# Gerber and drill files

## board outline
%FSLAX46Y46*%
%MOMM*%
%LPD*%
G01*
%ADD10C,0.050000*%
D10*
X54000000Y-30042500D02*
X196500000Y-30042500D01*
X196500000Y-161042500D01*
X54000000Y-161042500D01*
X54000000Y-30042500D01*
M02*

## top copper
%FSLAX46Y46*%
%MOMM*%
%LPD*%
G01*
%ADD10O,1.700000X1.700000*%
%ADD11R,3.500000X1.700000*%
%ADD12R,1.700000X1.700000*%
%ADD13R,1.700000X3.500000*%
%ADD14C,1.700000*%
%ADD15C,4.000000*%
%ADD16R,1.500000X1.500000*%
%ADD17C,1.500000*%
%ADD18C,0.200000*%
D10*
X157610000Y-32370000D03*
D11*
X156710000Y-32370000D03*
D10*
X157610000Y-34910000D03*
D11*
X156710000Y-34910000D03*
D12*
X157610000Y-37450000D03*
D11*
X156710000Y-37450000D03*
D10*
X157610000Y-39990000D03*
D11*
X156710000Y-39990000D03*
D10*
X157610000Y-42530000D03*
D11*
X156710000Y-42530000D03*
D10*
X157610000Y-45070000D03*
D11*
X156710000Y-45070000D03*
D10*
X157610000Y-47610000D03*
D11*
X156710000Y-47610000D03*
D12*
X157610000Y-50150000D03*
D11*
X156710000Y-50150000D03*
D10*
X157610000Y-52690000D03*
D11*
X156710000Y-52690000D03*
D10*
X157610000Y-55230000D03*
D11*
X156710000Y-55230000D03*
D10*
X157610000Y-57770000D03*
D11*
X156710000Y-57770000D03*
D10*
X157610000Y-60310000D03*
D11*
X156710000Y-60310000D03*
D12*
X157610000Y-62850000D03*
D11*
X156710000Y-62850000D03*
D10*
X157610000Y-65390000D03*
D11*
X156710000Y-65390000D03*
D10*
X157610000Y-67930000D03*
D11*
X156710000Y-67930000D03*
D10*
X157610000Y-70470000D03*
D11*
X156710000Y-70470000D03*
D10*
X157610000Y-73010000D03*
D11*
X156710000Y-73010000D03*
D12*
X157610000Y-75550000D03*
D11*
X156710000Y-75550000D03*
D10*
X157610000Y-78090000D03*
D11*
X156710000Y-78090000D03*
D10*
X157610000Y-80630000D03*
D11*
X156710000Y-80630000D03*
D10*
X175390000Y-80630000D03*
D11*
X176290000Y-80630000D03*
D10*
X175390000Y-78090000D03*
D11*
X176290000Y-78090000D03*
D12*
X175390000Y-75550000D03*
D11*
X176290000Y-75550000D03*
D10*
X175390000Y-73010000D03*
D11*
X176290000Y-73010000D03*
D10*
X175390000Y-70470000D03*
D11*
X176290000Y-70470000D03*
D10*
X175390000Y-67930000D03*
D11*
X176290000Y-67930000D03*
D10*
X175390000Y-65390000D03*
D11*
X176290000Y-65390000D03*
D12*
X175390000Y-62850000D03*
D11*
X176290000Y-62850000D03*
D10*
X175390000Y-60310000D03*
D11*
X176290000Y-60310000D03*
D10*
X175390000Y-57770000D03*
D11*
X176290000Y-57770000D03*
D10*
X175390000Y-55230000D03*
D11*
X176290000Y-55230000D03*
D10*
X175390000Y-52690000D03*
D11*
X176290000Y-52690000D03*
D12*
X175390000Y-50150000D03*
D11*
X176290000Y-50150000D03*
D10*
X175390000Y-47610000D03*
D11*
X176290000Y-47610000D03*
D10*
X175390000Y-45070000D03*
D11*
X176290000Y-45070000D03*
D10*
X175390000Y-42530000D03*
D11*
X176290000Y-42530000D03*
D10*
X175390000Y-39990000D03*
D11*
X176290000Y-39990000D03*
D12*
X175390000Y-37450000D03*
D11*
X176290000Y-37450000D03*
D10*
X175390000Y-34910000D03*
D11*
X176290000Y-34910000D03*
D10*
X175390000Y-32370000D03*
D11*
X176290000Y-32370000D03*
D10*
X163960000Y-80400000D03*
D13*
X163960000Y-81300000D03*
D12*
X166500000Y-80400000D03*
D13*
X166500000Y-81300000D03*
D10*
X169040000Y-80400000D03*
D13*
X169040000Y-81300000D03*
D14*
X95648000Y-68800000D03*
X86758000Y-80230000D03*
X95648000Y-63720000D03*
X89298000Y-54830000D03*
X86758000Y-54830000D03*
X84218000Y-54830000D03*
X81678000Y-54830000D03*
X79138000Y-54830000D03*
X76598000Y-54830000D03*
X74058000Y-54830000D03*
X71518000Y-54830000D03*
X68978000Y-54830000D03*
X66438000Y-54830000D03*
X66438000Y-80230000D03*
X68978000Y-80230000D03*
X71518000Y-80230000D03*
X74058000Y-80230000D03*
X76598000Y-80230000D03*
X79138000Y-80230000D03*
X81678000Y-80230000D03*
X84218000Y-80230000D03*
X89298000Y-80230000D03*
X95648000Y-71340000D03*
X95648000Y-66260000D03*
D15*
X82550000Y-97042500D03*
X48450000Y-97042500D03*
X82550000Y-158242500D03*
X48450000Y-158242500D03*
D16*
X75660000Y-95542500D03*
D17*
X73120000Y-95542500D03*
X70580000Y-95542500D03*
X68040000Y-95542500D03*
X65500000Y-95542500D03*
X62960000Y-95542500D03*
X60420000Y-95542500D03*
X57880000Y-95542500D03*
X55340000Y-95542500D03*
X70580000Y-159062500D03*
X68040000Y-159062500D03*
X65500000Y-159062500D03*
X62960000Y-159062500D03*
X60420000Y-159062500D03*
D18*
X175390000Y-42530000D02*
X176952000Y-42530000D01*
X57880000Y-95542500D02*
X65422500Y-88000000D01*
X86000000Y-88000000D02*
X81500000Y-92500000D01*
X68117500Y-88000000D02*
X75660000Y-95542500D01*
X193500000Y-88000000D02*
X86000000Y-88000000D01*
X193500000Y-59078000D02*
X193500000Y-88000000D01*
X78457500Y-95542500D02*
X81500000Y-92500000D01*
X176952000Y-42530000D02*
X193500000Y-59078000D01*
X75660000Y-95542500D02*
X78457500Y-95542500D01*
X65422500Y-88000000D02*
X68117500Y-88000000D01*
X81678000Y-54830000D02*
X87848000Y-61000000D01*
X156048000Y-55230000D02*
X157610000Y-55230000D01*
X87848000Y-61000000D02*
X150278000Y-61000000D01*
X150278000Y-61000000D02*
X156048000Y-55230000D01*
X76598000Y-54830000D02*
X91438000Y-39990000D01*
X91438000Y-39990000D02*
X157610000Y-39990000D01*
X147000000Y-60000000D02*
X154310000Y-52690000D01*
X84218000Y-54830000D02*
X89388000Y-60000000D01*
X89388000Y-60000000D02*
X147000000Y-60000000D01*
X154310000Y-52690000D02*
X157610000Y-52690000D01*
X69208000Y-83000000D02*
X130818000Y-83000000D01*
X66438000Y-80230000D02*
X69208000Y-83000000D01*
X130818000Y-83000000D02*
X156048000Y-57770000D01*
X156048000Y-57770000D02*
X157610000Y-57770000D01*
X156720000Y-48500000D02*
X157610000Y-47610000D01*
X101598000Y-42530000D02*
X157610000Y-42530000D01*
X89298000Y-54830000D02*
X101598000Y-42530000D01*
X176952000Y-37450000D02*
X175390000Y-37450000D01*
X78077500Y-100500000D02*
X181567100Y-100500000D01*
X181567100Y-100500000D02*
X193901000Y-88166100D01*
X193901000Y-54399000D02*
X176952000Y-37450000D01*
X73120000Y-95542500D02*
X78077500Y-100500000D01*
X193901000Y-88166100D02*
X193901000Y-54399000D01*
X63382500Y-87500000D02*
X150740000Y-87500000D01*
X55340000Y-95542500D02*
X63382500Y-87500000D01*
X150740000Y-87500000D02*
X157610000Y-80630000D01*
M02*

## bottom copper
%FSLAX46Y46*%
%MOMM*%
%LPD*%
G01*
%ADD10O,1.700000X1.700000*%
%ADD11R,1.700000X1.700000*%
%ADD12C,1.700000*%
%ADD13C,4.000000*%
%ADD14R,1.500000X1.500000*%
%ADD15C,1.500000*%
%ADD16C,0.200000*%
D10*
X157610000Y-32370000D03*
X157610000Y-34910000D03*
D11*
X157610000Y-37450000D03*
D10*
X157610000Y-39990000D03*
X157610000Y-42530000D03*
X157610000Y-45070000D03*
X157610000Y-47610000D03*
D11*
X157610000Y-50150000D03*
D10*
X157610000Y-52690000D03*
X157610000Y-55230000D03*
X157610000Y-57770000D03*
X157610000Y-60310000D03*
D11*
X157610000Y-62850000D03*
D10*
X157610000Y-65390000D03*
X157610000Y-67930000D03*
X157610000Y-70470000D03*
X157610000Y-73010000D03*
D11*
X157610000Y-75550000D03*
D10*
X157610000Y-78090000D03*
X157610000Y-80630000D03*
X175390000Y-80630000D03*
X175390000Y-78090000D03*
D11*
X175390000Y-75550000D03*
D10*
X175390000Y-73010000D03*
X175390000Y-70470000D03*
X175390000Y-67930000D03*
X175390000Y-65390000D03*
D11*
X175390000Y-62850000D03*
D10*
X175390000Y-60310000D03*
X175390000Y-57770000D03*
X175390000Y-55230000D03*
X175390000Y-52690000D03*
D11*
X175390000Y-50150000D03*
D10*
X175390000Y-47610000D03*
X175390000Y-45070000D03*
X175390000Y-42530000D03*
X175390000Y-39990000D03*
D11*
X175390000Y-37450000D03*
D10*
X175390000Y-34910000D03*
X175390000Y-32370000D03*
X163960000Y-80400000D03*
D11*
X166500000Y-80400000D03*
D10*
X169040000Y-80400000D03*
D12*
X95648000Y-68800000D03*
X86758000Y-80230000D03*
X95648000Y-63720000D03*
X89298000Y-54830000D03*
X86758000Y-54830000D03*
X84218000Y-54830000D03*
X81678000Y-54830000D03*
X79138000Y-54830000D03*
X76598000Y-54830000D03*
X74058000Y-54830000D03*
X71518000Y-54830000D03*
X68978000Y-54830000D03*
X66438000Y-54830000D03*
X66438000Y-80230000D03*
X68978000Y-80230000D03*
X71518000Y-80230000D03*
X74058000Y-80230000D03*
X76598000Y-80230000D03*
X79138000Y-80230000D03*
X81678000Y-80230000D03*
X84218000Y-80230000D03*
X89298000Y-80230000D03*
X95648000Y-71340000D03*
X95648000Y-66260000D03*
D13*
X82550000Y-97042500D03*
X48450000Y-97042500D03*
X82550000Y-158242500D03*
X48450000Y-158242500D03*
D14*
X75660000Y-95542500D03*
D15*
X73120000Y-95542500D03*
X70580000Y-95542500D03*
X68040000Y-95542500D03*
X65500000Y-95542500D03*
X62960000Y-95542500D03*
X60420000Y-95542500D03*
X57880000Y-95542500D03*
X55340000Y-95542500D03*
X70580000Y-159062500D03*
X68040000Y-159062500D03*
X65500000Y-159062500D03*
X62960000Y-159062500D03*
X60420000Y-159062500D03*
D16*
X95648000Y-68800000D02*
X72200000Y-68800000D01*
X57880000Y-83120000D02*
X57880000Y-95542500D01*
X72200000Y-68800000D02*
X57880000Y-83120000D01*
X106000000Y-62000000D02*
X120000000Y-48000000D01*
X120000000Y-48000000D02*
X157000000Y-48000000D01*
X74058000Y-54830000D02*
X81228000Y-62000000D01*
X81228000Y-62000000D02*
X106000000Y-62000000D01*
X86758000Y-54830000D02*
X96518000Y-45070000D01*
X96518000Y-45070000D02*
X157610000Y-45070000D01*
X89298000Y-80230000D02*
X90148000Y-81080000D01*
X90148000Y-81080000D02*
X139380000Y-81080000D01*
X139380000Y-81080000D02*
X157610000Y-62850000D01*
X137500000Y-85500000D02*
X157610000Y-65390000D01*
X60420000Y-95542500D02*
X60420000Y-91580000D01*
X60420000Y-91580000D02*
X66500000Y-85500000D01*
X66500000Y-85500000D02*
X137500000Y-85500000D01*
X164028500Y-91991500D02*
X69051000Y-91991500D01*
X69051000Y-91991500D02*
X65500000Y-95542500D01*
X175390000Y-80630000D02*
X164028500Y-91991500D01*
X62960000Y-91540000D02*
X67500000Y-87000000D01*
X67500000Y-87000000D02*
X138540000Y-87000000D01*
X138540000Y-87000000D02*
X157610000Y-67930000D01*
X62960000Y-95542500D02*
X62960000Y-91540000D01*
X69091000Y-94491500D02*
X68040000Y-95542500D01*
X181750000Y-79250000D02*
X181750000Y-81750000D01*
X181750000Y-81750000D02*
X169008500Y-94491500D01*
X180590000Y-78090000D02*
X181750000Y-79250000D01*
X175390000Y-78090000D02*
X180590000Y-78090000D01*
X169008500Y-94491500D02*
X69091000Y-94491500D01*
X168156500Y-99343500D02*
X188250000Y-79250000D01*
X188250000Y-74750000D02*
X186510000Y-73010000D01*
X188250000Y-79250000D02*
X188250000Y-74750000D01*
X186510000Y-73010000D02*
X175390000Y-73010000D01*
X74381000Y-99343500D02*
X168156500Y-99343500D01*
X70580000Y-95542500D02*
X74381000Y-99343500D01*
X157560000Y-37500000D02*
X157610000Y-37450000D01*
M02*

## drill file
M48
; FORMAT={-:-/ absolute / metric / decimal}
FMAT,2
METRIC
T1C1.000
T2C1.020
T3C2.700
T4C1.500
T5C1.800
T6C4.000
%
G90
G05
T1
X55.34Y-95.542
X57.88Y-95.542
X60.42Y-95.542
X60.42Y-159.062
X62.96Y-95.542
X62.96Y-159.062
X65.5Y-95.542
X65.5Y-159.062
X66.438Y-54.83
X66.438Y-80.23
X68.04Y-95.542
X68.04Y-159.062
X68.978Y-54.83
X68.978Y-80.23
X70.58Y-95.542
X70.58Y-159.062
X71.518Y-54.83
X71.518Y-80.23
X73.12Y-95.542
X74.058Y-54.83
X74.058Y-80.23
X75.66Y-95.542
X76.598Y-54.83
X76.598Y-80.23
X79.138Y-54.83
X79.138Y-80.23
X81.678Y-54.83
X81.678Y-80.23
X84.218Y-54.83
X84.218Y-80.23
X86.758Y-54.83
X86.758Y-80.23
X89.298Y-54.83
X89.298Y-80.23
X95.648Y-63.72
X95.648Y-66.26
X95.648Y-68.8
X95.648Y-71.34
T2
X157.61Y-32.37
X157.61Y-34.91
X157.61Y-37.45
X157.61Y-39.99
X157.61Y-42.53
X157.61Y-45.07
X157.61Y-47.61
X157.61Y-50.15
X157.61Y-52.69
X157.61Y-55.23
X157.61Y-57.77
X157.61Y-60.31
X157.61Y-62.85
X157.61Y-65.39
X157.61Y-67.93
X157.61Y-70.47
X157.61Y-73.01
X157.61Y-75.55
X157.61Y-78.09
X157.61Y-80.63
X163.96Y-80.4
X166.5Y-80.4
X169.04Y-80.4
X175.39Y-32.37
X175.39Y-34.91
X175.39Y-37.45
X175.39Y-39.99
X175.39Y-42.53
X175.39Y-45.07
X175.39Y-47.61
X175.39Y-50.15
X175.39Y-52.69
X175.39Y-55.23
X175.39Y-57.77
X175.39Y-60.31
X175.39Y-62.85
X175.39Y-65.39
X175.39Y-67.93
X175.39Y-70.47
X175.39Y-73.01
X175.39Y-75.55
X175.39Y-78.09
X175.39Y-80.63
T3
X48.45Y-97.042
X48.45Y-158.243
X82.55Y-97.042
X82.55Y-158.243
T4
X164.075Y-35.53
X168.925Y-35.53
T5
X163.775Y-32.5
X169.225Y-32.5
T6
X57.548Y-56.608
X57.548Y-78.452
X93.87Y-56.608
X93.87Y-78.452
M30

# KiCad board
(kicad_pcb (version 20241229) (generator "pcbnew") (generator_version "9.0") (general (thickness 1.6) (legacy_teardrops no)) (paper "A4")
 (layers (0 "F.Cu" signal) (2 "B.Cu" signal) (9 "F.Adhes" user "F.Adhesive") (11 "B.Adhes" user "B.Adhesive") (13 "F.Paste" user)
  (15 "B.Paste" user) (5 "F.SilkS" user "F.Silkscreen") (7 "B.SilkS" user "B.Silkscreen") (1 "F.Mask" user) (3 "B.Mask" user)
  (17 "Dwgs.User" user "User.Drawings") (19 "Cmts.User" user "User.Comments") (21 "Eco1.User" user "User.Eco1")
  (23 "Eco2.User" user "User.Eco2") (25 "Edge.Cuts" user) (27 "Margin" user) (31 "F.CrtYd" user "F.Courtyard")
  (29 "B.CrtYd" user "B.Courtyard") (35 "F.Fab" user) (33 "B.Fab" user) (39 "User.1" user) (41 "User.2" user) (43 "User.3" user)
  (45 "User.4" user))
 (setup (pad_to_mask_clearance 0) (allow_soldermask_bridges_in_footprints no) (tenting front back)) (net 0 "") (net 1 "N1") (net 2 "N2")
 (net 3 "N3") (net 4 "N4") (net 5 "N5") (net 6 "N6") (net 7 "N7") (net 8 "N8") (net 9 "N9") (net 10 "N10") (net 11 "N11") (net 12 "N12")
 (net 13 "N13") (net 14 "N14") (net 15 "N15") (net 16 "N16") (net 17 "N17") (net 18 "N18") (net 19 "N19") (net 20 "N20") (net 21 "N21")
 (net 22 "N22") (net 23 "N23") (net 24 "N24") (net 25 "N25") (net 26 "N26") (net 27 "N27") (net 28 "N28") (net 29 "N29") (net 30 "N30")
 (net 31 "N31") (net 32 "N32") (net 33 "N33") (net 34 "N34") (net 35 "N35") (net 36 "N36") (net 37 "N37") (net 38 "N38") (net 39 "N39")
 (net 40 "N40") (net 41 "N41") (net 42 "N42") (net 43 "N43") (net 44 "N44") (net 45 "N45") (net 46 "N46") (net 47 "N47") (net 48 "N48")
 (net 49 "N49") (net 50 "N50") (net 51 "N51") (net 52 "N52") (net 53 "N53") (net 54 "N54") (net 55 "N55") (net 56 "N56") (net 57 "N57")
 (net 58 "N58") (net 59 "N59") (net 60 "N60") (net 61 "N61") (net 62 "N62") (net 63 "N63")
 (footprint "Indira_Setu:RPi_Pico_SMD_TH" (layer "F.Cu") (at 166.5 56.5)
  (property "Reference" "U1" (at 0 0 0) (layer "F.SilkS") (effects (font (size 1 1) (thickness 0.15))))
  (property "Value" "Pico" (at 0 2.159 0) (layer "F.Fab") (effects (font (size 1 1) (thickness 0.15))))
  (pad "" np_thru_hole oval (at -2.725 -24) (size 1.8 1.8) (drill 1.8) (layers "*.Cu" "*.Mask"))
  (pad "" np_thru_hole oval (at -2.425 -20.97) (size 1.5 1.5) (drill 1.5) (layers "*.Cu" "*.Mask"))
  (pad "" np_thru_hole oval (at 2.425 -20.97) (size 1.5 1.5) (drill 1.5) (layers "*.Cu" "*.Mask"))
  (pad "" np_thru_hole oval (at 2.725 -24) (size 1.8 1.8) (drill 1.8) (layers "*.Cu" "*.Mask"))
  (pad "1" thru_hole oval (at -8.89 -24.13) (size 1.7 1.7) (drill 1.02) (layers "*.Cu" "*.Mask") (remove_unused_layers no) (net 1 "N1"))
  (pad "1" smd rect (at -8.89 -24.13) (size 3.5 1.7) (drill (offset -0.9 0)) (layers "F.Cu" "F.Mask") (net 1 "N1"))
  (pad "2" thru_hole oval (at -8.89 -21.59) (size 1.7 1.7) (drill 1.02) (layers "*.Cu" "*.Mask") (remove_unused_layers no) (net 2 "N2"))
  (pad "2" smd rect (at -8.89 -21.59) (size 3.5 1.7) (drill (offset -0.9 0)) (layers "F.Cu" "F.Mask") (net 2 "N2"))
  (pad "3" thru_hole rect (at -8.89 -19.05) (size 1.7 1.7) (drill 1.02) (layers "*.Cu" "*.Mask") (remove_unused_layers no) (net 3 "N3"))
  (pad "3" smd rect (at -8.89 -19.05) (size 3.5 1.7) (drill (offset -0.9 0)) (layers "F.Cu" "F.Mask") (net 3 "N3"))
  (pad "4" thru_hole oval (at -8.89 -16.51) (size 1.7 1.7) (drill 1.02) (layers "*.Cu" "*.Mask") (remove_unused_layers no) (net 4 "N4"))
  (pad "4" smd rect (at -8.89 -16.51) (size 3.5 1.7) (drill (offset -0.9 0)) (layers "F.Cu" "F.Mask") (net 4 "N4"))
  (pad "5" thru_hole oval (at -8.89 -13.97) (size 1.7 1.7) (drill 1.02) (layers "*.Cu" "*.Mask") (remove_unused_layers no) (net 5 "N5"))
  (pad "5" smd rect (at -8.89 -13.97) (size 3.5 1.7) (drill (offset -0.9 0)) (layers "F.Cu" "F.Mask") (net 5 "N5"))
  (pad "6" thru_hole oval (at -8.89 -11.43) (size 1.7 1.7) (drill 1.02) (layers "*.Cu" "*.Mask") (remove_unused_layers no) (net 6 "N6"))
  (pad "6" smd rect (at -8.89 -11.43) (size 3.5 1.7) (drill (offset -0.9 0)) (layers "F.Cu" "F.Mask") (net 6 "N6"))
  (pad "7" thru_hole oval (at -8.89 -8.89) (size 1.7 1.7) (drill 1.02) (layers "*.Cu" "*.Mask") (remove_unused_layers no) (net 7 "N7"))
  (pad "7" smd rect (at -8.89 -8.89) (size 3.5 1.7) (drill (offset -0.9 0)) (layers "F.Cu" "F.Mask") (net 7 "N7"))
  (pad "8" thru_hole rect (at -8.89 -6.35) (size 1.7 1.7) (drill 1.02) (layers "*.Cu" "*.Mask") (remove_unused_layers no) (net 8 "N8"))
  (pad "8" smd rect (at -8.89 -6.35) (size 3.5 1.7) (drill (offset -0.9 0)) (layers "F.Cu" "F.Mask") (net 8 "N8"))
  (pad "9" thru_hole oval (at -8.89 -3.81) (size 1.7 1.7) (drill 1.02) (layers "*.Cu" "*.Mask") (remove_unused_layers no) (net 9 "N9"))
  (pad "9" smd rect (at -8.89 -3.81) (size 3.5 1.7) (drill (offset -0.9 0)) (layers "F.Cu" "F.Mask") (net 9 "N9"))
  (pad "10" thru_hole oval (at -8.89 -1.27) (size 1.7 1.7) (drill 1.02) (layers "*.Cu" "*.Mask") (remove_unused_layers no) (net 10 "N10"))
  (pad "10" smd rect (at -8.89 -1.27) (size 3.5 1.7) (drill (offset -0.9 0)) (layers "F.Cu" "F.Mask") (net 10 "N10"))
  (pad "11" thru_hole oval (at -8.89 1.27) (size 1.7 1.7) (drill 1.02) (layers "*.Cu" "*.Mask") (remove_unused_layers no) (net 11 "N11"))
  (pad "11" smd rect (at -8.89 1.27) (size 3.5 1.7) (drill (offset -0.9 0)) (layers "F.Cu" "F.Mask") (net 11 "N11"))
  (pad "12" thru_hole oval (at -8.89 3.81) (size 1.7 1.7) (drill 1.02) (layers "*.Cu" "*.Mask") (remove_unused_layers no) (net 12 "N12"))
  (pad "12" smd rect (at -8.89 3.81) (size 3.5 1.7) (drill (offset -0.9 0)) (layers "F.Cu" "F.Mask") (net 12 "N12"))
  (pad "13" thru_hole rect (at -8.89 6.35) (size 1.7 1.7) (drill 1.02) (layers "*.Cu" "*.Mask") (remove_unused_layers no) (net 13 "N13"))
  (pad "13" smd rect (at -8.89 6.35) (size 3.5 1.7) (drill (offset -0.9 0)) (layers "F.Cu" "F.Mask") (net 13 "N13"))
  (pad "14" thru_hole oval (at -8.89 8.89) (size 1.7 1.7) (drill 1.02) (layers "*.Cu" "*.Mask") (remove_unused_layers no) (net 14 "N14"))
  (pad "14" smd rect (at -8.89 8.89) (size 3.5 1.7) (drill (offset -0.9 0)) (layers "F.Cu" "F.Mask") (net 14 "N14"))
  (pad "15" thru_hole oval (at -8.89 11.43) (size 1.7 1.7) (drill 1.02) (layers "*.Cu" "*.Mask") (remove_unused_layers no) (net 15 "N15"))
  (pad "15" smd rect (at -8.89 11.43) (size 3.5 1.7) (drill (offset -0.9 0)) (layers "F.Cu" "F.Mask") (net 15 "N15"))
  (pad "16" thru_hole oval (at -8.89 13.97) (size 1.7 1.7) (drill 1.02) (layers "*.Cu" "*.Mask") (remove_unused_layers no) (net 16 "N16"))
  (pad "16" smd rect (at -8.89 13.97) (size 3.5 1.7) (drill (offset -0.9 0)) (layers "F.Cu" "F.Mask") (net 16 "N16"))
  (pad "17" thru_hole oval (at -8.89 16.51) (size 1.7 1.7) (drill 1.02) (layers "*.Cu" "*.Mask") (remove_unused_layers no) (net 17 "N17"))
  (pad "17" smd rect (at -8.89 16.51) (size 3.5 1.7) (drill (offset -0.9 0)) (layers "F.Cu" "F.Mask") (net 17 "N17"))
  (pad "18" thru_hole rect (at -8.89 19.05) (size 1.7 1.7) (drill 1.02) (layers "*.Cu" "*.Mask") (remove_unused_layers no) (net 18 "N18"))
  (pad "18" smd rect (at -8.89 19.05) (size 3.5 1.7) (drill (offset -0.9 0)) (layers "F.Cu" "F.Mask") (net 18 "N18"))
  (pad "19" thru_hole oval (at -8.89 21.59) (size 1.7 1.7) (drill 1.02) (layers "*.Cu" "*.Mask") (remove_unused_layers no) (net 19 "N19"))
  (pad "19" smd rect (at -8.89 21.59) (size 3.5 1.7) (drill (offset -0.9 0)) (layers "F.Cu" "F.Mask") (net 19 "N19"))
  (pad "20" thru_hole oval (at -8.89 24.13) (size 1.7 1.7) (drill 1.02) (layers "*.Cu" "*.Mask") (remove_unused_layers no) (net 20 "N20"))
  (pad "20" smd rect (at -8.89 24.13) (size 3.5 1.7) (drill (offset -0.9 0)) (layers "F.Cu" "F.Mask") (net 20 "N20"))
  (pad "21" thru_hole oval (at 8.89 24.13) (size 1.7 1.7) (drill 1.02) (layers "*.Cu" "*.Mask") (remove_unused_layers no) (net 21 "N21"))
  (pad "21" smd rect (at 8.89 24.13) (size 3.5 1.7) (drill (offset 0.9 0)) (layers "F.Cu" "F.Mask") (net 21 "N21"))
  (pad "22" thru_hole oval (at 8.89 21.59) (size 1.7 1.7) (drill 1.02) (layers "*.Cu" "*.Mask") (remove_unused_layers no) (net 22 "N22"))
  (pad "22" smd rect (at 8.89 21.59) (size 3.5 1.7) (drill (offset 0.9 0)) (layers "F.Cu" "F.Mask") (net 22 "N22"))
  (pad "23" thru_hole rect (at 8.89 19.05) (size 1.7 1.7) (drill 1.02) (layers "*.Cu" "*.Mask") (remove_unused_layers no) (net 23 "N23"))
  (pad "23" smd rect (at 8.89 19.05) (size 3.5 1.7) (drill (offset 0.9 0)) (layers "F.Cu" "F.Mask") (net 23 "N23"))
  (pad "24" thru_hole oval (at 8.89 16.51) (size 1.7 1.7) (drill 1.02) (layers "*.Cu" "*.Mask") (remove_unused_layers no) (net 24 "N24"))
  (pad "24" smd rect (at 8.89 16.51) (size 3.5 1.7) (drill (offset 0.9 0)) (layers "F.Cu" "F.Mask") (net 24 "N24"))
  (pad "25" thru_hole oval (at 8.89 13.97) (size 1.7 1.7) (drill 1.02) (layers "*.Cu" "*.Mask") (remove_unused_layers no) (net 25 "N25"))
  (pad "25" smd rect (at 8.89 13.97) (size 3.5 1.7) (drill (offset 0.9 0)) (layers "F.Cu" "F.Mask") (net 25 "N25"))
  (pad "26" thru_hole oval (at 8.89 11.43) (size 1.7 1.7) (drill 1.02) (layers "*.Cu" "*.Mask") (remove_unused_layers no) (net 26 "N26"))
  (pad "26" smd rect (at 8.89 11.43) (size 3.5 1.7) (drill (offset 0.9 0)) (layers "F.Cu" "F.Mask") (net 26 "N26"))
  (pad "27" thru_hole oval (at 8.89 8.89) (size 1.7 1.7) (drill 1.02) (layers "*.Cu" "*.Mask") (remove_unused_layers no) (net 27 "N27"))
  (pad "27" smd rect (at 8.89 8.89) (size 3.5 1.7) (drill (offset 0.9 0)) (layers "F.Cu" "F.Mask") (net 27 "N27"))
  (pad "28" thru_hole rect (at 8.89 6.35) (size 1.7 1.7) (drill 1.02) (layers "*.Cu" "*.Mask") (remove_unused_layers no) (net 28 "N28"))
  (pad "28" smd rect (at 8.89 6.35) (size 3.5 1.7) (drill (offset 0.9 0)) (layers "F.Cu" "F.Mask") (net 28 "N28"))
  (pad "29" thru_hole oval (at 8.89 3.81) (size 1.7 1.7) (drill 1.02) (layers "*.Cu" "*.Mask") (remove_unused_layers no) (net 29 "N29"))
  (pad "29" smd rect (at 8.89 3.81) (size 3.5 1.7) (drill (offset 0.9 0)) (layers "F.Cu" "F.Mask") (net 29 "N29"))
  (pad "30" thru_hole oval (at 8.89 1.27) (size 1.7 1.7) (drill 1.02) (layers "*.Cu" "*.Mask") (remove_unused_layers no) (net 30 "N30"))
  (pad "30" smd rect (at 8.89 1.27) (size 3.5 1.7) (drill (offset 0.9 0)) (layers "F.Cu" "F.Mask") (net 30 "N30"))
  (pad "31" thru_hole oval (at 8.89 -1.27) (size 1.7 1.7) (drill 1.02) (layers "*.Cu" "*.Mask") (remove_unused_layers no) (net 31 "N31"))
  (pad "31" smd rect (at 8.89 -1.27) (size 3.5 1.7) (drill (offset 0.9 0)) (layers "F.Cu" "F.Mask") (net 31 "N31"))
  (pad "32" thru_hole oval (at 8.89 -3.81) (size 1.7 1.7) (drill 1.02) (layers "*.Cu" "*.Mask") (remove_unused_layers no) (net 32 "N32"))
  (pad "32" smd rect (at 8.89 -3.81) (size 3.5 1.7) (drill (offset 0.9 0)) (layers "F.Cu" "F.Mask") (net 32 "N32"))
  (pad "33" thru_hole rect (at 8.89 -6.35) (size 1.7 1.7) (drill 1.02) (layers "*.Cu" "*.Mask") (remove_unused_layers no) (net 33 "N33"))
  (pad "33" smd rect (at 8.89 -6.35) (size 3.5 1.7) (drill (offset 0.9 0)) (layers "F.Cu" "F.Mask") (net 33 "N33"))
  (pad "34" thru_hole oval (at 8.89 -8.89) (size 1.7 1.7) (drill 1.02) (layers "*.Cu" "*.Mask") (remove_unused_layers no) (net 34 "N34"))
  (pad "34" smd rect (at 8.89 -8.89) (size 3.5 1.7) (drill (offset 0.9 0)) (layers "F.Cu" "F.Mask") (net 34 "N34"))
  (pad "35" thru_hole oval (at 8.89 -11.43) (size 1.7 1.7) (drill 1.02) (layers "*.Cu" "*.Mask") (remove_unused_layers no) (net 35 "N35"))
  (pad "35" smd rect (at 8.89 -11.43) (size 3.5 1.7) (drill (offset 0.9 0)) (layers "F.Cu" "F.Mask") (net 35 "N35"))
  (pad "36" thru_hole oval (at 8.89 -13.97) (size 1.7 1.7) (drill 1.02) (layers "*.Cu" "*.Mask") (remove_unused_layers no) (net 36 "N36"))
  (pad "36" smd rect (at 8.89 -13.97) (size 3.5 1.7) (drill (offset 0.9 0)) (layers "F.Cu" "F.Mask") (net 36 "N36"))
  (pad "37" thru_hole oval (at 8.89 -16.51) (size 1.7 1.7) (drill 1.02) (layers "*.Cu" "*.Mask") (remove_unused_layers no) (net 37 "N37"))
  (pad "37" smd rect (at 8.89 -16.51) (size 3.5 1.7) (drill (offset 0.9 0)) (layers "F.Cu" "F.Mask") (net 37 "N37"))
  (pad "38" thru_hole rect (at 8.89 -19.05) (size 1.7 1.7) (drill 1.02) (layers "*.Cu" "*.Mask") (remove_unused_layers no) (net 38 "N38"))
  (pad "38" smd rect (at 8.89 -19.05) (size 3.5 1.7) (drill (offset 0.9 0)) (layers "F.Cu" "F.Mask") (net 38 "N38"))
  (pad "39" thru_hole oval (at 8.89 -21.59) (size 1.7 1.7) (drill 1.02) (layers "*.Cu" "*.Mask") (remove_unused_layers no) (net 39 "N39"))
  (pad "39" smd rect (at 8.89 -21.59) (size 3.5 1.7) (drill (offset 0.9 0)) (layers "F.Cu" "F.Mask") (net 39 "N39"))
  (pad "40" thru_hole oval (at 8.89 -24.13) (size 1.7 1.7) (drill 1.02) (layers "*.Cu" "*.Mask") (remove_unused_layers no) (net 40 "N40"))
  (pad "40" smd rect (at 8.89 -24.13) (size 3.5 1.7) (drill (offset 0.9 0)) (layers "F.Cu" "F.Mask") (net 40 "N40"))
  (pad "41" thru_hole oval (at -2.54 23.9) (size 1.7 1.7) (drill 1.02) (layers "*.Cu" "*.Mask") (remove_unused_layers no) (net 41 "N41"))
  (pad "41" smd rect (at -2.54 23.9 90) (size 3.5 1.7) (drill (offset -0.9 0)) (layers "F.Cu" "F.Mask") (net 41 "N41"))
  (pad "42" thru_hole rect (at 0 23.9) (size 1.7 1.7) (drill 1.02) (layers "*.Cu" "*.Mask") (remove_unused_layers no) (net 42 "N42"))
  (pad "42" smd rect (at 0 23.9 90) (size 3.5 1.7) (drill (offset -0.9 0)) (layers "F.Cu" "F.Mask") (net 42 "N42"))
  (pad "43" thru_hole oval (at 2.54 23.9) (size 1.7 1.7) (drill 1.02) (layers "*.Cu" "*.Mask") (remove_unused_layers no) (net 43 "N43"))
  (pad "43" smd rect (at 2.54 23.9 90) (size 3.5 1.7) (drill (offset -0.9 0)) (layers "F.Cu" "F.Mask") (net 43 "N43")))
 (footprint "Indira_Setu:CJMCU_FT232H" (layer "F.Cu") (at 54.5 81.5 90)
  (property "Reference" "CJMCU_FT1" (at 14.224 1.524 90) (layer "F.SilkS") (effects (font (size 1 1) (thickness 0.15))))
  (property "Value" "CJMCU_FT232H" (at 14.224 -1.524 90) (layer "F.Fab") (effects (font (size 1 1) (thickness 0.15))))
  (pad "" np_thru_hole circle (at 3.048 3.048 90) (size 4 4) (drill 4) (layers "*.Cu" "*.Mask"))
  (pad "" np_thru_hole circle (at 3.048 39.37 90) (size 4 4) (drill 4) (layers "*.Cu" "*.Mask"))
  (pad "" np_thru_hole circle (at 24.892 3.048 90) (size 4 4) (drill 4) (layers "*.Cu" "*.Mask"))
  (pad "" np_thru_hole circle (at 24.892 39.37 90) (size 4 4) (drill 4) (layers "*.Cu" "*.Mask"))
  (pad "+3.3V" thru_hole circle (at 12.7 41.148 90) (size 1.7 1.7) (drill 1) (layers "*.Cu" "*.Mask") (remove_unused_layers no)
   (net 36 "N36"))
  (pad "+5V1" thru_hole circle (at 1.27 32.258 90) (size 1.7 1.7) (drill 1) (layers "*.Cu" "*.Mask") (remove_unused_layers no)
   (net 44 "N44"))
  (pad "+5V2" thru_hole circle (at 17.78 41.148 90) (size 1.7 1.7) (drill 1) (layers "*.Cu" "*.Mask") (remove_unused_layers no)
   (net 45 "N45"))
  (pad "AC0" thru_hole circle (at 26.67 34.798 90) (size 1.7 1.7) (drill 1) (layers "*.Cu" "*.Mask") (remove_unused_layers no) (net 5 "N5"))
  (pad "AC1" thru_hole circle (at 26.67 32.258 90) (size 1.7 1.7) (drill 1) (layers "*.Cu" "*.Mask") (remove_unused_layers no) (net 6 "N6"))
  (pad "AC2" thru_hole circle (at 26.67 29.718 90) (size 1.7 1.7) (drill 1) (layers "*.Cu" "*.Mask") (remove_unused_layers no) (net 9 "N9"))
  (pad "AC3" thru_hole circle (at 26.67 27.178 90) (size 1.7 1.7) (drill 1) (layers "*.Cu" "*.Mask") (remove_unused_layers no)
   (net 10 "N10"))
  (pad "AC4" thru_hole circle (at 26.67 24.638 90) (size 1.7 1.7) (drill 1) (layers "*.Cu" "*.Mask") (remove_unused_layers no)
   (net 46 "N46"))
  (pad "AC5" thru_hole circle (at 26.67 22.098 90) (size 1.7 1.7) (drill 1) (layers "*.Cu" "*.Mask") (remove_unused_layers no) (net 4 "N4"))
  (pad "AC6" thru_hole circle (at 26.67 19.558 90) (size 1.7 1.7) (drill 1) (layers "*.Cu" "*.Mask") (remove_unused_layers no) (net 7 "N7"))
  (pad "AC7" thru_hole circle (at 26.67 17.018 90) (size 1.7 1.7) (drill 1) (layers "*.Cu" "*.Mask") (remove_unused_layers no)
   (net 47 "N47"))
  (pad "AC8" thru_hole circle (at 26.67 14.478 90) (size 1.7 1.7) (drill 1) (layers "*.Cu" "*.Mask") (remove_unused_layers no)
   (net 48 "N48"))
  (pad "AC9" thru_hole circle (at 26.67 11.938 90) (size 1.7 1.7) (drill 1) (layers "*.Cu" "*.Mask") (remove_unused_layers no)
   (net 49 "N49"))
  (pad "AD0" thru_hole circle (at 1.27 11.938 90) (size 1.7 1.7) (drill 1) (layers "*.Cu" "*.Mask") (remove_unused_layers no) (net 11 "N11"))
  (pad "AD1" thru_hole circle (at 1.27 14.478 90) (size 1.7 1.7) (drill 1) (layers "*.Cu" "*.Mask") (remove_unused_layers no) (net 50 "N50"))
  (pad "AD2" thru_hole circle (at 1.27 17.018 90) (size 1.7 1.7) (drill 1) (layers "*.Cu" "*.Mask") (remove_unused_layers no) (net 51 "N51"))
  (pad "AD3" thru_hole circle (at 1.27 19.558 90) (size 1.7 1.7) (drill 1) (layers "*.Cu" "*.Mask") (remove_unused_layers no) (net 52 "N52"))
  (pad "AD4" thru_hole circle (at 1.27 22.098 90) (size 1.7 1.7) (drill 1) (layers "*.Cu" "*.Mask") (remove_unused_layers no) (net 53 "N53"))
  (pad "AD5" thru_hole circle (at 1.27 24.638 90) (size 1.7 1.7) (drill 1) (layers "*.Cu" "*.Mask") (remove_unused_layers no) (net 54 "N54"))
  (pad "AD6" thru_hole circle (at 1.27 27.178 90) (size 1.7 1.7) (drill 1) (layers "*.Cu" "*.Mask") (remove_unused_layers no) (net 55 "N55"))
  (pad "AD7" thru_hole circle (at 1.27 29.718 90) (size 1.7 1.7) (drill 1) (layers "*.Cu" "*.Mask") (remove_unused_layers no) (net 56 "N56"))
  (pad "GND1" thru_hole circle (at 1.27 34.798 90) (size 1.7 1.7) (drill 1) (layers "*.Cu" "*.Mask") (remove_unused_layers no)
   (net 13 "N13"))
  (pad "GND2" thru_hole circle (at 10.16 41.148 90) (size 1.7 1.7) (drill 1) (layers "*.Cu" "*.Mask") (remove_unused_layers no)
   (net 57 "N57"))
  (pad "Vcore" thru_hole circle (at 15.24 41.148 90) (size 1.7 1.7) (drill 1) (layers "*.Cu" "*.Mask") (remove_unused_layers no)
   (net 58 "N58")))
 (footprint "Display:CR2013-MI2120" (layer "F.Cu") (at 75.66 95.5425 -90)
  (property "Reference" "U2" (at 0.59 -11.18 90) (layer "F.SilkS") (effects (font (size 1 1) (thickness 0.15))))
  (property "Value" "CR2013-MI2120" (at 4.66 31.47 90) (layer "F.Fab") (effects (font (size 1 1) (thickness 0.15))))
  (pad "" thru_hole circle (at 1.5 -6.89 270) (size 4 4) (drill 2.7) (layers "*.Cu" "*.Mask") (remove_unused_layers no))
  (pad "" thru_hole circle (at 1.5 27.21 270) (size 4 4) (drill 2.7) (layers "*.Cu" "*.Mask") (remove_unused_layers no))
  (pad "" thru_hole circle (at 62.7 -6.89 270) (size 4 4) (drill 2.7) (layers "*.Cu" "*.Mask") (remove_unused_layers no))
  (pad "" thru_hole circle (at 62.7 27.21 270) (size 4 4) (drill 2.7) (layers "*.Cu" "*.Mask") (remove_unused_layers no))
  (pad "1" thru_hole rect (at 0 0 270) (size 1.5 1.5) (drill 1) (layers "*.Cu" "*.Mask") (remove_unused_layers no) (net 36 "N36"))
  (pad "2" thru_hole circle (at 0 2.54 270) (size 1.5 1.5) (drill 1) (layers "*.Cu" "*.Mask") (remove_unused_layers no) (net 38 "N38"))
  (pad "3" thru_hole circle (at 0 5.08 270) (size 1.5 1.5) (drill 1) (layers "*.Cu" "*.Mask") (remove_unused_layers no) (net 24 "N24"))
  (pad "4" thru_hole circle (at 0 7.62 270) (size 1.5 1.5) (drill 1) (layers "*.Cu" "*.Mask") (remove_unused_layers no) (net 22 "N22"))
  (pad "5" thru_hole circle (at 0 10.16 270) (size 1.5 1.5) (drill 1) (layers "*.Cu" "*.Mask") (remove_unused_layers no) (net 21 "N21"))
  (pad "6" thru_hole circle (at 0 12.7 270) (size 1.5 1.5) (drill 1) (layers "*.Cu" "*.Mask") (remove_unused_layers no) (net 15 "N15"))
  (pad "7" thru_hole circle (at 0 15.24 270) (size 1.5 1.5) (drill 1) (layers "*.Cu" "*.Mask") (remove_unused_layers no) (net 14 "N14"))
  (pad "8" thru_hole circle (at 0 17.78 270) (size 1.5 1.5) (drill 1) (layers "*.Cu" "*.Mask") (remove_unused_layers no) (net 36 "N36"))
  (pad "9" thru_hole circle (at 0 20.32 270) (size 1.5 1.5) (drill 1) (layers "*.Cu" "*.Mask") (remove_unused_layers no) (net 20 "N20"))
  (pad "10" thru_hole circle (at 63.52 5.08 270) (size 1.5 1.5) (drill 1) (layers "*.Cu" "*.Mask") (remove_unused_layers no) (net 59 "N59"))
  (pad "11" thru_hole circle (at 63.52 7.62 270) (size 1.5 1.5) (drill 1) (layers "*.Cu" "*.Mask") (remove_unused_layers no) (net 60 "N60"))
  (pad "12" thru_hole circle (at 63.52 10.16 270) (size 1.5 1.5) (drill 1) (layers "*.Cu" "*.Mask") (remove_unused_layers no) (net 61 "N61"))
  (pad "13" thru_hole circle (at 63.52 12.7 270) (size 1.5 1.5) (drill 1) (layers "*.Cu" "*.Mask") (remove_unused_layers no) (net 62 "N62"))
  (pad "14" thru_hole circle (at 63.52 15.24 270) (size 1.5 1.5) (drill 1) (layers "*.Cu" "*.Mask") (remove_unused_layers no) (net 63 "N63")))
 (gr_rect (start 54 30.0425) (end 196.5 161.0425) (stroke (width 0.05) (type default)) (fill no) (layer "Edge.Cuts"))
 (segment (start 175.39 42.53) (end 176.952 42.53) (width 0.2) (layer "F.Cu") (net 36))
 (segment (start 57.88 95.5425) (end 65.4225 88) (width 0.2) (layer "F.Cu") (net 36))
 (segment (start 86 88) (end 81.5 92.5) (width 0.2) (layer "F.Cu") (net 36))
 (segment (start 68.1175 88) (end 75.66 95.5425) (width 0.2) (layer "F.Cu") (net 36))
 (segment (start 193.5 88) (end 86 88) (width 0.2) (layer "F.Cu") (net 36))
 (segment (start 193.5 59.078) (end 193.5 88) (width 0.2) (layer "F.Cu") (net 36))
 (segment (start 78.4575 95.5425) (end 81.5 92.5) (width 0.2) (layer "F.Cu") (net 36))
 (segment (start 176.952 42.53) (end 193.5 59.078) (width 0.2) (layer "F.Cu") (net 36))
 (segment (start 75.66 95.5425) (end 78.4575 95.5425) (width 0.2) (layer "F.Cu") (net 36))
 (segment (start 65.4225 88) (end 68.1175 88) (width 0.2) (layer "F.Cu") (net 36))
 (segment (start 95.648 68.8) (end 72.2 68.8) (width 0.2) (layer "B.Cu") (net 36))
 (segment (start 57.88 83.12) (end 57.88 95.5425) (width 0.2) (layer "B.Cu") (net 36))
 (segment (start 72.2 68.8) (end 57.88 83.12) (width 0.2) (layer "B.Cu") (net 36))
 (segment (start 81.678 54.83) (end 87.848 61) (width 0.2) (layer "F.Cu") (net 10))
 (segment (start 156.048 55.23) (end 157.61 55.23) (width 0.2) (layer "F.Cu") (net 10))
 (segment (start 87.848 61) (end 150.278 61) (width 0.2) (layer "F.Cu") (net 10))
 (segment (start 150.278 61) (end 156.048 55.23) (width 0.2) (layer "F.Cu") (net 10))
 (segment (start 76.598 54.83) (end 91.438 39.99) (width 0.2) (layer "F.Cu") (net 4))
 (segment (start 91.438 39.99) (end 157.61 39.99) (width 0.2) (layer "F.Cu") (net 4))
 (segment (start 147 60) (end 154.31 52.69) (width 0.2) (layer "F.Cu") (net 9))
 (segment (start 84.218 54.83) (end 89.388 60) (width 0.2) (layer "F.Cu") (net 9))
 (segment (start 89.388 60) (end 147 60) (width 0.2) (layer "F.Cu") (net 9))
 (segment (start 154.31 52.69) (end 157.61 52.69) (width 0.2) (layer "F.Cu") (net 9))
 (segment (start 69.208 83) (end 130.818 83) (width 0.2) (layer "F.Cu") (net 11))
 (segment (start 66.438 80.23) (end 69.208 83) (width 0.2) (layer "F.Cu") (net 11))
 (segment (start 130.818 83) (end 156.048 57.77) (width 0.2) (layer "F.Cu") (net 11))
 (segment (start 156.048 57.77) (end 157.61 57.77) (width 0.2) (layer "F.Cu") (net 11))
 (segment (start 156.72 48.5) (end 157.61 47.61) (width 0.2) (layer "F.Cu") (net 7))
 (segment (start 106 62) (end 120 48) (width 0.2) (layer "B.Cu") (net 7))
 (segment (start 120 48) (end 157 48) (width 0.2) (layer "B.Cu") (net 7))
 (segment (start 74.058 54.83) (end 81.228 62) (width 0.2) (layer "B.Cu") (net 7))
 (segment (start 81.228 62) (end 106 62) (width 0.2) (layer "B.Cu") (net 7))
 (segment (start 101.598 42.53) (end 157.61 42.53) (width 0.2) (layer "F.Cu") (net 5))
 (segment (start 89.298 54.83) (end 101.598 42.53) (width 0.2) (layer "F.Cu") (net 5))
 (segment (start 86.758 54.83) (end 96.518 45.07) (width 0.2) (layer "B.Cu") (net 6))
 (segment (start 96.518 45.07) (end 157.61 45.07) (width 0.2) (layer "B.Cu") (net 6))
 (segment (start 89.298 80.23) (end 90.148 81.08) (width 0.2) (layer "B.Cu") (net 13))
 (segment (start 90.148 81.08) (end 139.38 81.08) (width 0.2) (layer "B.Cu") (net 13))
 (segment (start 139.38 81.08) (end 157.61 62.85) (width 0.2) (layer "B.Cu") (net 13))
 (segment (start 137.5 85.5) (end 157.61 65.39) (width 0.2) (layer "B.Cu") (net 14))
 (segment (start 60.42 95.5425) (end 60.42 91.58) (width 0.2) (layer "B.Cu") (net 14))
 (segment (start 60.42 91.58) (end 66.5 85.5) (width 0.2) (layer "B.Cu") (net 14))
 (segment (start 66.5 85.5) (end 137.5 85.5) (width 0.2) (layer "B.Cu") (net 14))
 (segment (start 164.0285 91.9915) (end 69.051 91.9915) (width 0.2) (layer "B.Cu") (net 21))
 (segment (start 69.051 91.9915) (end 65.5 95.5425) (width 0.2) (layer "B.Cu") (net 21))
 (segment (start 175.39 80.63) (end 164.0285 91.9915) (width 0.2) (layer "B.Cu") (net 21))
 (segment (start 176.952 37.45) (end 175.39 37.45) (width 0.2) (layer "F.Cu") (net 38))
 (segment (start 78.0775 100.5) (end 181.5671 100.5) (width 0.2) (layer "F.Cu") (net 38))
 (segment (start 181.5671 100.5) (end 193.901 88.1661) (width 0.2) (layer "F.Cu") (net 38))
 (segment (start 193.901 54.399) (end 176.952 37.45) (width 0.2) (layer "F.Cu") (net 38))
 (segment (start 73.12 95.5425) (end 78.0775 100.5) (width 0.2) (layer "F.Cu") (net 38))
 (segment (start 193.901 88.1661) (end 193.901 54.399) (width 0.2) (layer "F.Cu") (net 38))
 (segment (start 62.96 91.54) (end 67.5 87) (width 0.2) (layer "B.Cu") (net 15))
 (segment (start 67.5 87) (end 138.54 87) (width 0.2) (layer "B.Cu") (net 15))
 (segment (start 138.54 87) (end 157.61 67.93) (width 0.2) (layer "B.Cu") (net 15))
 (segment (start 62.96 95.5425) (end 62.96 91.54) (width 0.2) (layer "B.Cu") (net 15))
 (segment (start 69.091 94.4915) (end 68.04 95.5425) (width 0.2) (layer "B.Cu") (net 22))
 (segment (start 181.75 79.25) (end 181.75 81.75) (width 0.2) (layer "B.Cu") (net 22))
 (segment (start 181.75 81.75) (end 169.0085 94.4915) (width 0.2) (layer "B.Cu") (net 22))
 (segment (start 180.59 78.09) (end 181.75 79.25) (width 0.2) (layer "B.Cu") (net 22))
 (segment (start 175.39 78.09) (end 180.59 78.09) (width 0.2) (layer "B.Cu") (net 22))
 (segment (start 169.0085 94.4915) (end 69.091 94.4915) (width 0.2) (layer "B.Cu") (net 22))
 (segment (start 168.1565 99.3435) (end 188.25 79.25) (width 0.2) (layer "B.Cu") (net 24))
 (segment (start 188.25 74.75) (end 186.51 73.01) (width 0.2) (layer "B.Cu") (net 24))
 (segment (start 188.25 79.25) (end 188.25 74.75) (width 0.2) (layer "B.Cu") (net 24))
 (segment (start 186.51 73.01) (end 175.39 73.01) (width 0.2) (layer "B.Cu") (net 24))
 (segment (start 74.381 99.3435) (end 168.1565 99.3435) (width 0.2) (layer "B.Cu") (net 24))
 (segment (start 70.58 95.5425) (end 74.381 99.3435) (width 0.2) (layer "B.Cu") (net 24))
 (segment (start 63.3825 87.5) (end 150.74 87.5) (width 0.2) (layer "F.Cu") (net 20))
 (segment (start 55.34 95.5425) (end 63.3825 87.5) (width 0.2) (layer "F.Cu") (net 20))
 (segment (start 150.74 87.5) (end 157.61 80.63) (width 0.2) (layer "F.Cu") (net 20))
 (segment (start 157.56 37.5) (end 157.61 37.45) (width 0.2) (layer "B.Cu") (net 3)))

